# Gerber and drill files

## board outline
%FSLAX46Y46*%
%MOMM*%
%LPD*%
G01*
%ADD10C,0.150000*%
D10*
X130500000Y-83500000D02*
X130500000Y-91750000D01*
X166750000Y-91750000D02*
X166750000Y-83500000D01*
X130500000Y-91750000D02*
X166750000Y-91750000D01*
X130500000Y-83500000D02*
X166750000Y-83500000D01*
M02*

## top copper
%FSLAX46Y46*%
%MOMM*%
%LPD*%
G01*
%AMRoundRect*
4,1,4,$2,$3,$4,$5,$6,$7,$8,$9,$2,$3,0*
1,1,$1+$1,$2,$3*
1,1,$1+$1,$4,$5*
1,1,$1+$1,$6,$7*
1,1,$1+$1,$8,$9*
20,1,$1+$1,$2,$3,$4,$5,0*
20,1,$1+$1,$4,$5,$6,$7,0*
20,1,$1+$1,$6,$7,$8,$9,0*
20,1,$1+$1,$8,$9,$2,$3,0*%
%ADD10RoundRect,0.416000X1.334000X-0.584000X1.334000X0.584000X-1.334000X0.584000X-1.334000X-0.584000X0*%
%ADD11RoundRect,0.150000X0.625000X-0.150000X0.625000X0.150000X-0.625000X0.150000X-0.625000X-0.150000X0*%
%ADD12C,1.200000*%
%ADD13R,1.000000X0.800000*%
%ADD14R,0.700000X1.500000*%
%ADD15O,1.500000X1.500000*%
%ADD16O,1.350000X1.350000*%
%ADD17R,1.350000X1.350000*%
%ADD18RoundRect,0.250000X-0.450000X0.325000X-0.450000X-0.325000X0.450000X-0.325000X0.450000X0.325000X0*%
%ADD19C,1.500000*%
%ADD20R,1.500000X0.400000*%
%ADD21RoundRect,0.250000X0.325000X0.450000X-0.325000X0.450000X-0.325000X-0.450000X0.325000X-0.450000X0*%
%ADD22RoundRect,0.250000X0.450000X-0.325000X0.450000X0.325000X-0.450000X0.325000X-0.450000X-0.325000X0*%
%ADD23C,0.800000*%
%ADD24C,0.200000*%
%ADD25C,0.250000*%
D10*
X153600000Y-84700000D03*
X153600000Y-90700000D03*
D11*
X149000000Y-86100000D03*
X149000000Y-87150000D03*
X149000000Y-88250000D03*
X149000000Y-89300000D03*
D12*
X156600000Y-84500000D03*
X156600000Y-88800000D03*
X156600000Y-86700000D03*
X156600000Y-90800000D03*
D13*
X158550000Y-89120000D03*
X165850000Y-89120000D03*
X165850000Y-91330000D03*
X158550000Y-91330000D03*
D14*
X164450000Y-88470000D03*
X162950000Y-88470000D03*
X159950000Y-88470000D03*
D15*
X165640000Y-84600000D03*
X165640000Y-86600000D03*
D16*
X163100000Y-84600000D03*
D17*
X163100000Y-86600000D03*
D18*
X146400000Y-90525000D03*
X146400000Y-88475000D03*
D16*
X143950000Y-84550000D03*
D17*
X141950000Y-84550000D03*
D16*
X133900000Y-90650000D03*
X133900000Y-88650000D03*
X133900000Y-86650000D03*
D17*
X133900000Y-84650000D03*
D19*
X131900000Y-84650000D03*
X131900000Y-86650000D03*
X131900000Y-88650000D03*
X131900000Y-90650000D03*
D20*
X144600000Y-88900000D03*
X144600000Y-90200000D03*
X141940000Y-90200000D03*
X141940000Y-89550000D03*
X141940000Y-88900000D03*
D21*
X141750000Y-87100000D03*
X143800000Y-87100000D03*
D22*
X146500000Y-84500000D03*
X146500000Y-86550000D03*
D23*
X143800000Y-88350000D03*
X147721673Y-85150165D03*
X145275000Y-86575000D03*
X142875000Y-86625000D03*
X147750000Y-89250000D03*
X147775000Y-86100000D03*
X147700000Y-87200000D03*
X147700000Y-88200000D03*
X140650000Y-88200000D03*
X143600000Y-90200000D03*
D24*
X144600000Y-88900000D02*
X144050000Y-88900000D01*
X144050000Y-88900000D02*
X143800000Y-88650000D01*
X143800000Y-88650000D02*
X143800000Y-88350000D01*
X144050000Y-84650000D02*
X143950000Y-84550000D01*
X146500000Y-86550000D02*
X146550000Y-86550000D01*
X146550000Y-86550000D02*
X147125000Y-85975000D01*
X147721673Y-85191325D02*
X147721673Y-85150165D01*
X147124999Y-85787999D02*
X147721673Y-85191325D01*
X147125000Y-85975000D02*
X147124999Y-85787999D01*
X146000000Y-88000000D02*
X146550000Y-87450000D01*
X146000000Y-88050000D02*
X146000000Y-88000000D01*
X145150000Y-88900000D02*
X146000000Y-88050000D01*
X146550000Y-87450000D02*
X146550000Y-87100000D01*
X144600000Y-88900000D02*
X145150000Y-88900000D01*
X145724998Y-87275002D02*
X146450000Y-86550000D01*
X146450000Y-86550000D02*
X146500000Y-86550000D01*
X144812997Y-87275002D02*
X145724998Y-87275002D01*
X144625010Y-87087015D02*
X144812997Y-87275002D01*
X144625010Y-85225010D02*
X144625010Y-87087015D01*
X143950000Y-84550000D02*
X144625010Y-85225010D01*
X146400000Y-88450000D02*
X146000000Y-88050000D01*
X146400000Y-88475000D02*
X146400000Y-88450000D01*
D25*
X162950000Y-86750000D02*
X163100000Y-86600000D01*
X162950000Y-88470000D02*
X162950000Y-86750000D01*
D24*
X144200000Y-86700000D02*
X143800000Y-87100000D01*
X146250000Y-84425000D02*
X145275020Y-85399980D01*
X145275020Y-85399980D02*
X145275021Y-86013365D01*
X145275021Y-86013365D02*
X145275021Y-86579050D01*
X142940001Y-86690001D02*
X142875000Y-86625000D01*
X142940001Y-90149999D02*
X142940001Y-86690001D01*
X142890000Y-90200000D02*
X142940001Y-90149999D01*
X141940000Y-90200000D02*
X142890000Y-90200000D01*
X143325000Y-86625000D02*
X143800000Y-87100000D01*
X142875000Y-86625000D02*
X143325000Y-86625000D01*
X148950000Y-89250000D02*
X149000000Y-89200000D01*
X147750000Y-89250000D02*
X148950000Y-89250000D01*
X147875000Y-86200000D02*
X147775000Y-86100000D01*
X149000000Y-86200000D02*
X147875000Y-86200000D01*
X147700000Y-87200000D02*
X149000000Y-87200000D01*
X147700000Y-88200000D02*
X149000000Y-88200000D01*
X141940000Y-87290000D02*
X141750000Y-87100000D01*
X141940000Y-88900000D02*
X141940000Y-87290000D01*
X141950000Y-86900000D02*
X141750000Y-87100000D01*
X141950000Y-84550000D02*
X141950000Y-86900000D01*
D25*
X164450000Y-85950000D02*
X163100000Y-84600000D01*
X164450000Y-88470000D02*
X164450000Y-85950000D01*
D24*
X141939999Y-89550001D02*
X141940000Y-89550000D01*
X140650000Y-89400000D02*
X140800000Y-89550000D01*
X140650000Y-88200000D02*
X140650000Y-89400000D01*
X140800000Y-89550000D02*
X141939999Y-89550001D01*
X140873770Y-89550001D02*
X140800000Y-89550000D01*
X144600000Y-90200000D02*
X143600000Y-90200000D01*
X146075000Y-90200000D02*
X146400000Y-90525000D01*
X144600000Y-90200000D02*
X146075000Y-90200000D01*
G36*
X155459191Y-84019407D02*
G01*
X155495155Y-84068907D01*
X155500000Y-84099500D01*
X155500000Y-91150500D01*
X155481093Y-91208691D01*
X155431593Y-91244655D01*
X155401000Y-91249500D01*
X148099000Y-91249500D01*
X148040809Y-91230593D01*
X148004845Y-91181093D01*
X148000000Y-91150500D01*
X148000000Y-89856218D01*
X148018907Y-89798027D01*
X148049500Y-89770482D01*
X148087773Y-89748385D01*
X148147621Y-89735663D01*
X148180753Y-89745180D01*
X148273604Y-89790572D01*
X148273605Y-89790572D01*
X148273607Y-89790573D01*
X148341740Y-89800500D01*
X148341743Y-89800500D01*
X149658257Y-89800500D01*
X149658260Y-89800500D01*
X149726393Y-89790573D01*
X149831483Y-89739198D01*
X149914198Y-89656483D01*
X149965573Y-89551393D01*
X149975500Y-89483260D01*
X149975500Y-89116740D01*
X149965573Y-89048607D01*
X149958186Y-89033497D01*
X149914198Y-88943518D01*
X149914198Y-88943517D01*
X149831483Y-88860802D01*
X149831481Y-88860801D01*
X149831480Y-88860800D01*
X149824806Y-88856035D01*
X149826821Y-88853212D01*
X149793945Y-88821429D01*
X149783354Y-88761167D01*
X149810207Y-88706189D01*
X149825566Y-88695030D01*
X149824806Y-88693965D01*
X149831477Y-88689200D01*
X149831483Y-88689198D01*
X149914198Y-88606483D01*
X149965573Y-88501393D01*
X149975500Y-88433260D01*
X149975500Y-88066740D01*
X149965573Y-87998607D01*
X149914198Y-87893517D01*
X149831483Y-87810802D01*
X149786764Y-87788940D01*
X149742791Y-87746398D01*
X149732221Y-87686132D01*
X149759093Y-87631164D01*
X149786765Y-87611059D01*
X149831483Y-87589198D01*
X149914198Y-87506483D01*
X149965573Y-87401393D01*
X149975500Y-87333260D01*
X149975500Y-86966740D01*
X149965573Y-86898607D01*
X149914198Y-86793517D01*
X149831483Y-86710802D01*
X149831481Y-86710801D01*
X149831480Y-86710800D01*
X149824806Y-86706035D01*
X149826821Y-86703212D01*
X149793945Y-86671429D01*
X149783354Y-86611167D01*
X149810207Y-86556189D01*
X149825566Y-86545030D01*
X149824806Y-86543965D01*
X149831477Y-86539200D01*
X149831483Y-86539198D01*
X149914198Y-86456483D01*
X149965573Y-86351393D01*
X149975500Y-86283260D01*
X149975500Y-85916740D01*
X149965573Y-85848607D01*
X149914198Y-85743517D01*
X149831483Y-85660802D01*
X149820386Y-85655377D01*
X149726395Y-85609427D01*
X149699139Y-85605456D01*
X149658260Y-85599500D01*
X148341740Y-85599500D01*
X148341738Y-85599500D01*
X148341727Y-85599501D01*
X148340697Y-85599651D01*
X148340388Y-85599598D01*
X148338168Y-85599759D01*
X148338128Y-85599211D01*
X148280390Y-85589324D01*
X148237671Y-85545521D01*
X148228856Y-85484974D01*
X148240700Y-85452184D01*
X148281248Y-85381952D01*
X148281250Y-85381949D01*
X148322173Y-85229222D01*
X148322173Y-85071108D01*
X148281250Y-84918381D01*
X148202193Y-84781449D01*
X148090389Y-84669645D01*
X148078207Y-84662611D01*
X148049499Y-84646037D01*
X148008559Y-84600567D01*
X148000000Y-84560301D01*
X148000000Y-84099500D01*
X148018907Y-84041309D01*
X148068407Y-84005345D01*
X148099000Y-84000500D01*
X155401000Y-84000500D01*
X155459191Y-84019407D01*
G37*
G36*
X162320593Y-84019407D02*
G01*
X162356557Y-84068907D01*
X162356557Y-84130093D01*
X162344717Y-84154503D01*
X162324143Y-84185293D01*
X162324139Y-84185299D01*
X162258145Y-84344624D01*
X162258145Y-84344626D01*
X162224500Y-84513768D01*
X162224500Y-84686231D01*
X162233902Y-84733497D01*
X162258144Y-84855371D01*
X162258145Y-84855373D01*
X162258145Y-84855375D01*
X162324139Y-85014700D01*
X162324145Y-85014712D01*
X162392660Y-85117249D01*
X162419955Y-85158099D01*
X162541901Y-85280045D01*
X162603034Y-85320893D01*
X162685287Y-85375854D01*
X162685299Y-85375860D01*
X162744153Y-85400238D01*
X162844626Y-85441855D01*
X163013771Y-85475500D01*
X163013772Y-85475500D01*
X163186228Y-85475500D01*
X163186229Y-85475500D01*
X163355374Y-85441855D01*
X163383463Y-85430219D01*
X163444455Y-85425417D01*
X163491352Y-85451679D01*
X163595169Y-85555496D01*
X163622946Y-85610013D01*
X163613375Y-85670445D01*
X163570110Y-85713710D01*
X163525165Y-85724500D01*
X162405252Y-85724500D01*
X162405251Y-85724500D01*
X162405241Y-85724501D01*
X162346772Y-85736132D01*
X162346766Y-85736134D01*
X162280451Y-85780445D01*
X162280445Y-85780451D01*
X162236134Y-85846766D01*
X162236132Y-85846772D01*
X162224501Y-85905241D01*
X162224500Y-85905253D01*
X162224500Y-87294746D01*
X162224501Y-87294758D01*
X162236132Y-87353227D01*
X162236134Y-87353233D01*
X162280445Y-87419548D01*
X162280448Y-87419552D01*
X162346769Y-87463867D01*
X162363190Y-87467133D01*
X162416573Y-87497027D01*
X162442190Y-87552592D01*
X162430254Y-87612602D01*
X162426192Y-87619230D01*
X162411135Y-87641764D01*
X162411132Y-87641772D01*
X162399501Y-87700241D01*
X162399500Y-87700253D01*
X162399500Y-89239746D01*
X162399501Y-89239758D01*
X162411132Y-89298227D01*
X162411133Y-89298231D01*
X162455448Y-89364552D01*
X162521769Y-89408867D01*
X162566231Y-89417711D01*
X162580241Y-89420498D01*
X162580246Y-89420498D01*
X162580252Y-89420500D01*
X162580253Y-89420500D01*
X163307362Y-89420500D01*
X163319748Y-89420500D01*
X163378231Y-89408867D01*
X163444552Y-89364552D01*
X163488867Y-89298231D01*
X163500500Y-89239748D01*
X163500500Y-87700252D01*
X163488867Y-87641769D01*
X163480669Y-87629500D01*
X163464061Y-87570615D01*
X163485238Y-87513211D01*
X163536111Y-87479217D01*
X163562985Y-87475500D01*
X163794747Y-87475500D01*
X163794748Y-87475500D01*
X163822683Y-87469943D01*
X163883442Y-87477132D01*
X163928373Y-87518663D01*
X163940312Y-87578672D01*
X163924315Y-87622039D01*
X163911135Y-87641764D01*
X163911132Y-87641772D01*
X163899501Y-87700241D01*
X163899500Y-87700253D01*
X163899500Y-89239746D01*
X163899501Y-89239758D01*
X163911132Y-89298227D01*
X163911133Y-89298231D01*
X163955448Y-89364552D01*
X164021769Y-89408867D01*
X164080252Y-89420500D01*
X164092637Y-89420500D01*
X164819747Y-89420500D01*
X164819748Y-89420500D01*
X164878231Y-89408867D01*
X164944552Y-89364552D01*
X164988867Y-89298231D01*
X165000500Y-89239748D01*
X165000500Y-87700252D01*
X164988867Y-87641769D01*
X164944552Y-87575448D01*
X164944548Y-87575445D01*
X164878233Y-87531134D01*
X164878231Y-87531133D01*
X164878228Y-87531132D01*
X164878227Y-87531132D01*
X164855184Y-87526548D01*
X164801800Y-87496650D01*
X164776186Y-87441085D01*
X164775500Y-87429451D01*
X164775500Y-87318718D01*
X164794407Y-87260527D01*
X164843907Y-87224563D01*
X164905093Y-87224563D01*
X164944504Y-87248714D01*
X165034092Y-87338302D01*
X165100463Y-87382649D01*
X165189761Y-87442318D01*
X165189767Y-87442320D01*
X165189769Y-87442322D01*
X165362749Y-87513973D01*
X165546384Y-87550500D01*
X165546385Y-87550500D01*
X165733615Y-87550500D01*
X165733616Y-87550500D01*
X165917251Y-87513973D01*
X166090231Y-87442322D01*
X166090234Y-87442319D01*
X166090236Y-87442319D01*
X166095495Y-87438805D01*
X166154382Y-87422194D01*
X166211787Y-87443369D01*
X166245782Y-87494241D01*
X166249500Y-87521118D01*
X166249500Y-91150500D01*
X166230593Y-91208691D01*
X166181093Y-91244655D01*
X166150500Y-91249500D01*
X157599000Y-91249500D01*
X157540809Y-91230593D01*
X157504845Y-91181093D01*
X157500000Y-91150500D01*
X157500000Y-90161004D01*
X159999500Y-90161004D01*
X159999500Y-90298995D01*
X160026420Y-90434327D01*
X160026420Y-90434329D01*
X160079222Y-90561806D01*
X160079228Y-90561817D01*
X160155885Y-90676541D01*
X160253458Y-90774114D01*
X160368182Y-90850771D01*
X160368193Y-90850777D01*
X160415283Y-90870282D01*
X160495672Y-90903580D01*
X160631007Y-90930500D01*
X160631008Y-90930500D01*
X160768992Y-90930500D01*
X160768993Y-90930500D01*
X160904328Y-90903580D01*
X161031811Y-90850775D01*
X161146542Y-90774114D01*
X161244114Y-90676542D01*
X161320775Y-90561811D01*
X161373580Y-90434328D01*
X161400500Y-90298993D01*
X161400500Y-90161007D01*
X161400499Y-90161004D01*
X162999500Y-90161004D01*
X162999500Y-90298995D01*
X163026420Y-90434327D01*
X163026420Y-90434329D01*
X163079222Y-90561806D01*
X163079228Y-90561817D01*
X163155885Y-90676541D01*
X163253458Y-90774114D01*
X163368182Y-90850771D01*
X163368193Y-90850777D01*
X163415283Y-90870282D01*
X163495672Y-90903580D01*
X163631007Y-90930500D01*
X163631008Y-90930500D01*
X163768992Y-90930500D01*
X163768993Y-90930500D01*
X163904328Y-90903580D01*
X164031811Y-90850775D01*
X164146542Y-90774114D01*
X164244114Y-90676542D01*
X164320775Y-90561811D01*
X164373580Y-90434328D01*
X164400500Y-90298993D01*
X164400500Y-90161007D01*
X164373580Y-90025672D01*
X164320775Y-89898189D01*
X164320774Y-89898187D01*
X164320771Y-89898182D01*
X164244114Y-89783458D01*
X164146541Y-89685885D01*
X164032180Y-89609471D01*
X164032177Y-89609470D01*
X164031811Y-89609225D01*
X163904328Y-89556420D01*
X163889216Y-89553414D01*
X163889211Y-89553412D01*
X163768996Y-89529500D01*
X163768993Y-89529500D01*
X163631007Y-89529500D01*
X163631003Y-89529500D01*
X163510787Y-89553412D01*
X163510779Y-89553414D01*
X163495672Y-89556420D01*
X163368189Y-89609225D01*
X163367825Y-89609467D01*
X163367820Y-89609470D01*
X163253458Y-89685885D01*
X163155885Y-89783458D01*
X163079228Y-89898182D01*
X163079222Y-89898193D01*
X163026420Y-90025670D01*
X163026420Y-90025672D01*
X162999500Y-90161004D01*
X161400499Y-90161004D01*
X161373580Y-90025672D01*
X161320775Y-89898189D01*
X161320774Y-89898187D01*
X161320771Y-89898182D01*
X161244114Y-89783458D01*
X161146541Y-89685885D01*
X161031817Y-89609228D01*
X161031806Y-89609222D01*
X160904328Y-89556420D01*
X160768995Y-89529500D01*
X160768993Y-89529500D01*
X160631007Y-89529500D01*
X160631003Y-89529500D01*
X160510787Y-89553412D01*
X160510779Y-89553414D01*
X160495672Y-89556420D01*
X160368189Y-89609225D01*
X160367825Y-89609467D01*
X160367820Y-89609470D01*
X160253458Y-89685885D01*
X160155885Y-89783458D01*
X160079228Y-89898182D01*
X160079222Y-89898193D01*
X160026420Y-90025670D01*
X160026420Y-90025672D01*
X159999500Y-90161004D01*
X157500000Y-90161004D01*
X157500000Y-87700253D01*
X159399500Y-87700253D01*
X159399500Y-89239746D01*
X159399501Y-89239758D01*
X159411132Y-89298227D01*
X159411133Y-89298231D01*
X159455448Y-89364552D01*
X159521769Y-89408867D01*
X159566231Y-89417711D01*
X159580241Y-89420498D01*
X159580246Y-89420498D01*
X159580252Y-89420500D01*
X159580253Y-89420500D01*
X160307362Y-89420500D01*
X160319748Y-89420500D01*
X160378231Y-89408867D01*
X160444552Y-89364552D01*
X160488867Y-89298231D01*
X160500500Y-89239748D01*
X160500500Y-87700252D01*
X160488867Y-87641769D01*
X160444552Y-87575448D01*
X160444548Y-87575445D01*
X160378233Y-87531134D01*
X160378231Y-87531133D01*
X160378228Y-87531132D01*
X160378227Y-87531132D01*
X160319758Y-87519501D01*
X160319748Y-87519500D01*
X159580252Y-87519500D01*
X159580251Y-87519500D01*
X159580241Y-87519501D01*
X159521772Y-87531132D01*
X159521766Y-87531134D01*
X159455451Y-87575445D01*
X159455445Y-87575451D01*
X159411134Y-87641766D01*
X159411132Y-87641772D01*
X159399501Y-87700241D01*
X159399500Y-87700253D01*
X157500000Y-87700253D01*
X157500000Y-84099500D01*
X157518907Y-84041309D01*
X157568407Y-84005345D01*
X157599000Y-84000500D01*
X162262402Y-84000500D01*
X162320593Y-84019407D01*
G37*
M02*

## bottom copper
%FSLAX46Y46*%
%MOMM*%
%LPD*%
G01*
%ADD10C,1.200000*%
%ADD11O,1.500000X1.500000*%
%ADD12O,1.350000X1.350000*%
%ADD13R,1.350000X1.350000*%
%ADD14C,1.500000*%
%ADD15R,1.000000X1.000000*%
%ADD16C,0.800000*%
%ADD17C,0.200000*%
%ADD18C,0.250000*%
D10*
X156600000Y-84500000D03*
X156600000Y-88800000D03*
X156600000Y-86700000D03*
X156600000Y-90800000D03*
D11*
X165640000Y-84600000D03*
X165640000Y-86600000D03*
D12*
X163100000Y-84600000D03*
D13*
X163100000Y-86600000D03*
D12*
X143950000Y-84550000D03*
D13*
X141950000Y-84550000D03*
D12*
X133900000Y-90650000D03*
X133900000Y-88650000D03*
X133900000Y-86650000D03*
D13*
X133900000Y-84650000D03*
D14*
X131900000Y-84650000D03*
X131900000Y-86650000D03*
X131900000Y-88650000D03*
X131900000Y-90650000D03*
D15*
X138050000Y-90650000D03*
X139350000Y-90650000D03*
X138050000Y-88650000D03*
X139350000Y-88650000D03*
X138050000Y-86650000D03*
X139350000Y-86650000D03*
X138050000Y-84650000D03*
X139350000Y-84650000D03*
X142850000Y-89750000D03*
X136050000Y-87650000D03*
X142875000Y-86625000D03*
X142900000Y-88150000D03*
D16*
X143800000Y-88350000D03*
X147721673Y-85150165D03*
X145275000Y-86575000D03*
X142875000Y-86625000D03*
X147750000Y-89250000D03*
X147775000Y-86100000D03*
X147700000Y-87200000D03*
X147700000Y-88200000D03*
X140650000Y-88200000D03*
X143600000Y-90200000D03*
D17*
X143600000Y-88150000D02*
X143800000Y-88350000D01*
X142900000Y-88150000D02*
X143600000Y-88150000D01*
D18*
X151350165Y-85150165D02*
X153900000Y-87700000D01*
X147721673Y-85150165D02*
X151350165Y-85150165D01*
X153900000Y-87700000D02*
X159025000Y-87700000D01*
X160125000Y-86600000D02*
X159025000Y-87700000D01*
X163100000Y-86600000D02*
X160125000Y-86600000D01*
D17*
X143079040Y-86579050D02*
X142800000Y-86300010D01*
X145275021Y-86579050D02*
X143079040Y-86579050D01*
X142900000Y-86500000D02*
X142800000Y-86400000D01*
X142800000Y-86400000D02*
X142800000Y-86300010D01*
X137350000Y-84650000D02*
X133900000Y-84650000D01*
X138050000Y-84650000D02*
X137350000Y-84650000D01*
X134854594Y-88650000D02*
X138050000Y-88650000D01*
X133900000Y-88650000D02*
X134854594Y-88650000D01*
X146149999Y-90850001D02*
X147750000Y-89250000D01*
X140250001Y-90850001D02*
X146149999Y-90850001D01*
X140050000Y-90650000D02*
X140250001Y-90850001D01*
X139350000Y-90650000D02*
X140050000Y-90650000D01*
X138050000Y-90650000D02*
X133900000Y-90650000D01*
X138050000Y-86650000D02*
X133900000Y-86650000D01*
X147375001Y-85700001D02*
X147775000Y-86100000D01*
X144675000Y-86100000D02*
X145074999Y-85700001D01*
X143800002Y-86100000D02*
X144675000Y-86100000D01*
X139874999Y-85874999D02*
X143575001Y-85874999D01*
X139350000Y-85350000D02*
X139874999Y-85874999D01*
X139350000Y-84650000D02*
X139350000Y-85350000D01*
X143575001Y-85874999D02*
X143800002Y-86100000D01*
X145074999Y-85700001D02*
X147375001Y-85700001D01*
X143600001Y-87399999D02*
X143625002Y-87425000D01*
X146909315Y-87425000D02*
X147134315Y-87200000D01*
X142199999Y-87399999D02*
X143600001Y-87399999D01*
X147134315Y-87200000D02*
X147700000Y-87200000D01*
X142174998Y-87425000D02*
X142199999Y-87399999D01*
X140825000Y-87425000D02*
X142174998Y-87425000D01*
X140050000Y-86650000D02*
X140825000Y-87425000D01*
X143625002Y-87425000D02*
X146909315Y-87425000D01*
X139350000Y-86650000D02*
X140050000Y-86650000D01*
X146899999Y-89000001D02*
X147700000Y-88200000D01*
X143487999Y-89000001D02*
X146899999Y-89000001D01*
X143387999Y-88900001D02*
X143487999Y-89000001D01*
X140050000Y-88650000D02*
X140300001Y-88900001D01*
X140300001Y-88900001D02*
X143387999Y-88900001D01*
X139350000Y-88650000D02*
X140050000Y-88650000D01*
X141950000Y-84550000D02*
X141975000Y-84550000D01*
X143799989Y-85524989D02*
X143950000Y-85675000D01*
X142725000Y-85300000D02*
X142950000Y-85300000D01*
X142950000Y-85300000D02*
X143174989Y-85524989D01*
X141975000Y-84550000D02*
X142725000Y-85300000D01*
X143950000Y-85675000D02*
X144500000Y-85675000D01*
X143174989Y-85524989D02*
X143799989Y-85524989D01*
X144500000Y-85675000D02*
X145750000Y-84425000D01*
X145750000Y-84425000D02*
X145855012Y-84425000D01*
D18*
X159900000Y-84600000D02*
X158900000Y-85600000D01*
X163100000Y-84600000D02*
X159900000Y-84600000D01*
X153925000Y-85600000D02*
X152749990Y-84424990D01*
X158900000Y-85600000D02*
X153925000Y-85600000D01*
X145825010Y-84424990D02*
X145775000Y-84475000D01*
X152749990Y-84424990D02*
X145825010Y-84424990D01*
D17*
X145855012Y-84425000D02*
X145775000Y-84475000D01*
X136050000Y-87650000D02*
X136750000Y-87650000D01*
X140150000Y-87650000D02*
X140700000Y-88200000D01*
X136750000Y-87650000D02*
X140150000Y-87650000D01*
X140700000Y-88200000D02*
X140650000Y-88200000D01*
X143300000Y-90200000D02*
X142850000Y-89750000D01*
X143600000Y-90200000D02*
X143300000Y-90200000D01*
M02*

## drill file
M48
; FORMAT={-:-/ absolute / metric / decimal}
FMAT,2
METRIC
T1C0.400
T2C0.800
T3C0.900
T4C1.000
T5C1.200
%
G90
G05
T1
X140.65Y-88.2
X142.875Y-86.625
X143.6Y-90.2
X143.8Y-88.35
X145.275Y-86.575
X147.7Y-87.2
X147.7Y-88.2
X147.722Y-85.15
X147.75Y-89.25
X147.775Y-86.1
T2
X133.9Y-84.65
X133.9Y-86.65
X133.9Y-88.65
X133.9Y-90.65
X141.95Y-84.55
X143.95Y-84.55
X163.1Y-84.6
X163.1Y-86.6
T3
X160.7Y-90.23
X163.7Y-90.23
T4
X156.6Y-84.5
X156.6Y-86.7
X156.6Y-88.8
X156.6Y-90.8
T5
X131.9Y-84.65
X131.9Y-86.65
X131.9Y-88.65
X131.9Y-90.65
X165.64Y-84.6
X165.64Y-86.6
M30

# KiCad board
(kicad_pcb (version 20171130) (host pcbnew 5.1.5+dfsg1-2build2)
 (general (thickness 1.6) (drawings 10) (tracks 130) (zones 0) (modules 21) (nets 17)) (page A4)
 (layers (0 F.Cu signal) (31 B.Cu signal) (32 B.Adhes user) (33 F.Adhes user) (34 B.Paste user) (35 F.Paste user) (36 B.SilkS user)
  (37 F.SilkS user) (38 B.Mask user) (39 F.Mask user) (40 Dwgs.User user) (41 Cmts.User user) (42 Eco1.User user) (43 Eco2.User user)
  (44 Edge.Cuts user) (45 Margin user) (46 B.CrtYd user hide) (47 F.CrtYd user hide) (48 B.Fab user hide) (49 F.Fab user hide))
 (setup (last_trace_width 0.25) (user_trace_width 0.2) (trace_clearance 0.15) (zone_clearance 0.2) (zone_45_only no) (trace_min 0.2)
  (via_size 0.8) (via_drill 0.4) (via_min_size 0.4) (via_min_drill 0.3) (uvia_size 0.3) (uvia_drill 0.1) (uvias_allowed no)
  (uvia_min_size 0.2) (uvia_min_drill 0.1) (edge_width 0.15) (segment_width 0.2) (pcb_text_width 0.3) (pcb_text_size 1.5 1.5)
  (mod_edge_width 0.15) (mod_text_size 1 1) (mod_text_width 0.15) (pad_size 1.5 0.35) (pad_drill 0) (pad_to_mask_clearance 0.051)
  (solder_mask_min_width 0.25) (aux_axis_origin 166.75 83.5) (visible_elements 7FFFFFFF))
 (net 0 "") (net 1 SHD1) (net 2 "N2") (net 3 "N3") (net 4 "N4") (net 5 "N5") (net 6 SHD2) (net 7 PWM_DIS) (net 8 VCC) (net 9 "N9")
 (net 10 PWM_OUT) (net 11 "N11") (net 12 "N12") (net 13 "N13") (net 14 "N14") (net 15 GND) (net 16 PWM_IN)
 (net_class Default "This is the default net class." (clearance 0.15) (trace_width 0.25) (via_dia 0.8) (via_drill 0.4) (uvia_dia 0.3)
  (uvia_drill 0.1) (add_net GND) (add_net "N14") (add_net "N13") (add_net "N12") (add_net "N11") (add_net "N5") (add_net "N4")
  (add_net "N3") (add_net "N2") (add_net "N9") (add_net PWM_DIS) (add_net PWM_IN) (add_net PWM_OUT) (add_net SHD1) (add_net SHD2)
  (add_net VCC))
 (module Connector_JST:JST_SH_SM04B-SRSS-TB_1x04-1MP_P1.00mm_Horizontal (layer F.Cu) (at 151 87.7 90)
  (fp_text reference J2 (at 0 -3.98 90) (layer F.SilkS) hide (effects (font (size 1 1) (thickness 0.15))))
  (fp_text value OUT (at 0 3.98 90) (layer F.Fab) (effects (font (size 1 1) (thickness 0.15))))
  (pad MP smd roundrect (at 3 2.6 90) (size 2 3.5) (layers F.Cu F.Paste F.Mask) (roundrect_rratio 0.208) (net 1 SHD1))
  (pad MP smd roundrect (at -3 2.6 90) (size 2 3.5) (layers F.Cu F.Paste F.Mask) (roundrect_rratio 0.208) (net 1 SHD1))
  (pad 4 smd roundrect (at 1.6 -2 90) (size 0.6 1.55) (layers F.Cu F.Paste F.Mask) (roundrect_rratio 0.25) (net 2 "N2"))
  (pad 3 smd roundrect (at 0.55 -2 90) (size 0.6 1.55) (layers F.Cu F.Paste F.Mask) (roundrect_rratio 0.25) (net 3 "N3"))
  (pad 2 smd roundrect (at -0.55 -2 90) (size 0.6 1.55) (layers F.Cu F.Paste F.Mask) (roundrect_rratio 0.25) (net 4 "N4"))
  (pad 1 smd roundrect (at -1.6 -2 90) (size 0.6 1.55) (layers F.Cu F.Paste F.Mask) (roundrect_rratio 0.25) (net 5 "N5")))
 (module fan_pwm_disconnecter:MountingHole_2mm (layer F.Cu) (at 156.6 84.5)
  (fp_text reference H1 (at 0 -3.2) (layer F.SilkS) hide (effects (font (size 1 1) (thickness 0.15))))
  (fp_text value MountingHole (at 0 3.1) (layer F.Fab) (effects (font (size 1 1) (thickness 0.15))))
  (pad "" np_thru_hole circle (at 0 0) (size 1.2 1.2) (drill 1) (layers *.Cu *.Mask)))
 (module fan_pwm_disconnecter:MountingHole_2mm (layer F.Cu) (at 156.6 88.8)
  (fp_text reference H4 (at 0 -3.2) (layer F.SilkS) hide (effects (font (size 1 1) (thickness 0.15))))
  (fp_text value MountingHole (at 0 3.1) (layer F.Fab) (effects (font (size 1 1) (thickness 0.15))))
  (pad "" np_thru_hole circle (at 0 0) (size 1.2 1.2) (drill 1) (layers *.Cu *.Mask)))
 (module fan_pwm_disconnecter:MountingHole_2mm (layer F.Cu) (at 156.6 86.7)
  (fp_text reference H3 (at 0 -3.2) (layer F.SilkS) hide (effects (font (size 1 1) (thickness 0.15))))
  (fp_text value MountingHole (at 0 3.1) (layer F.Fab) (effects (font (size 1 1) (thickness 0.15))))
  (pad "" np_thru_hole circle (at 0 0) (size 1.2 1.2) (drill 1) (layers *.Cu *.Mask)))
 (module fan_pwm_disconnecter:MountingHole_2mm (layer F.Cu) (at 156.6 90.8)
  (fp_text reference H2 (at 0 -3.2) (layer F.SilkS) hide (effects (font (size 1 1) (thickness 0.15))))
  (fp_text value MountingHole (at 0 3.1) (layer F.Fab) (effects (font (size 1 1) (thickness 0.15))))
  (pad "" np_thru_hole circle (at 0 0) (size 1.2 1.2) (drill 1) (layers *.Cu *.Mask)))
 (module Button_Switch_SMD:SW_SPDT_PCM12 (layer F.Cu) (at 162.2 89.9)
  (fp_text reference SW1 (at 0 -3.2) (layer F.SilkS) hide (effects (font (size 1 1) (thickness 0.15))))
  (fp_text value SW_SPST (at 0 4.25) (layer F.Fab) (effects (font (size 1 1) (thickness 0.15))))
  (pad 4 smd rect (at -3.65 -0.78) (size 1 0.8) (layers F.Cu F.Paste F.Mask) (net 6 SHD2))
  (pad 4 smd rect (at 3.65 -0.78) (size 1 0.8) (layers F.Cu F.Paste F.Mask) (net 6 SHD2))
  (pad 4 smd rect (at 3.65 1.43) (size 1 0.8) (layers F.Cu F.Paste F.Mask) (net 6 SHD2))
  (pad 4 smd rect (at -3.65 1.43) (size 1 0.8) (layers F.Cu F.Paste F.Mask) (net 6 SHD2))
  (pad 3 smd rect (at 2.25 -1.43) (size 0.7 1.5) (layers F.Cu F.Paste F.Mask) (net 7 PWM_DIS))
  (pad 2 smd rect (at 0.75 -1.43) (size 0.7 1.5) (layers F.Cu F.Paste F.Mask) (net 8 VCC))
  (pad 1 smd rect (at -2.25 -1.43) (size 0.7 1.5) (layers F.Cu F.Paste F.Mask) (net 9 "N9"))
  (pad "" np_thru_hole circle (at 1.5 0.33) (size 0.9 0.9) (drill 0.9) (layers *.Cu *.Mask))
  (pad "" np_thru_hole circle (at -1.5 0.33) (size 0.9 0.9) (drill 0.9) (layers *.Cu *.Mask)))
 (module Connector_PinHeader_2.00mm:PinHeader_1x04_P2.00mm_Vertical (layer F.Cu) (at 163.1 86.6 180)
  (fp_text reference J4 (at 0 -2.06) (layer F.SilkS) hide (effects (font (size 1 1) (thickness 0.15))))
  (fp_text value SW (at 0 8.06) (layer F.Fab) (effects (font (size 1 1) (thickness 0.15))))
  (pad "" np_thru_hole oval (at -2.54 2 180) (size 1.5 1.5) (drill 1.2) (layers *.Cu *.Mask))
  (pad "" np_thru_hole oval (at -2.54 0 180) (size 1.5 1.5) (drill 1.2) (layers *.Cu *.Mask))
  (pad 2 thru_hole oval (at 0 2 180) (size 1.35 1.35) (drill 0.8) (layers *.Cu *.Mask) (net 7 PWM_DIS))
  (pad 1 thru_hole rect (at 0 0 180) (size 1.35 1.35) (drill 0.8) (layers *.Cu *.Mask) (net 8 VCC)))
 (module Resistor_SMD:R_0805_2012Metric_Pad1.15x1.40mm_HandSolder (layer F.Cu) (at 146.4 89.5 270)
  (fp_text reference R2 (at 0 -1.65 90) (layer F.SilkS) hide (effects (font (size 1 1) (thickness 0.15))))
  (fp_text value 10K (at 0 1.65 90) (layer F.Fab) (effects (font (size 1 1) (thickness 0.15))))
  (pad 2 smd roundrect (at 1.025 0 270) (size 1.15 1.4) (layers F.Cu F.Paste F.Mask) (roundrect_rratio 0.217391) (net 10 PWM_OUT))
  (pad 1 smd roundrect (at -1.025 0 270) (size 1.15 1.4) (layers F.Cu F.Paste F.Mask) (roundrect_rratio 0.217391) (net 8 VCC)))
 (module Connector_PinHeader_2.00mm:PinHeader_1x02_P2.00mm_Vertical (layer F.Cu) (at 141.95 84.55 90)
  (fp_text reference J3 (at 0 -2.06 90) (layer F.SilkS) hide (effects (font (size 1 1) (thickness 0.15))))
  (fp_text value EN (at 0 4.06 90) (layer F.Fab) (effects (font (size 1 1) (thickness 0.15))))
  (pad 2 thru_hole oval (at 0 2 90) (size 1.35 1.35) (drill 0.8) (layers *.Cu *.Mask) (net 8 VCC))
  (pad 1 thru_hole rect (at 0 0 90) (size 1.35 1.35) (drill 0.8) (layers *.Cu *.Mask) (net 7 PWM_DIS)))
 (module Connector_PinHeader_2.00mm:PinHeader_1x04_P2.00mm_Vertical (layer F.Cu) (at 133.9 84.65)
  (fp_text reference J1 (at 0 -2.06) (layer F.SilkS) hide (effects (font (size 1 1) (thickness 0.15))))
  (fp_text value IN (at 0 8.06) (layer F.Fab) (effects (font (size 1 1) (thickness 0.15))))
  (pad 4 thru_hole oval (at 0 6) (size 1.35 1.35) (drill 0.8) (layers *.Cu *.Mask) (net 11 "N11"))
  (pad 3 thru_hole oval (at 0 4) (size 1.35 1.35) (drill 0.8) (layers *.Cu *.Mask) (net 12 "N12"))
  (pad 2 thru_hole oval (at 0 2) (size 1.35 1.35) (drill 0.8) (layers *.Cu *.Mask) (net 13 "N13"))
  (pad 1 thru_hole rect (at 0 0) (size 1.35 1.35) (drill 0.8) (layers *.Cu *.Mask) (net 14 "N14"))
  (pad "" np_thru_hole circle (at -2 0) (size 1.5 1.5) (drill 1.2) (layers *.Cu *.Mask))
  (pad "" np_thru_hole circle (at -2 2) (size 1.5 1.5) (drill 1.2) (layers *.Cu *.Mask))
  (pad "" np_thru_hole circle (at -2 4) (size 1.5 1.5) (drill 1.2) (layers *.Cu *.Mask))
  (pad "" np_thru_hole circle (at -2 6) (size 1.5 1.5) (drill 1.2) (layers *.Cu *.Mask)))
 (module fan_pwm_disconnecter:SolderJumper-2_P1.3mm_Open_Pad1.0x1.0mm (layer B.Cu) (at 138.7 90.65)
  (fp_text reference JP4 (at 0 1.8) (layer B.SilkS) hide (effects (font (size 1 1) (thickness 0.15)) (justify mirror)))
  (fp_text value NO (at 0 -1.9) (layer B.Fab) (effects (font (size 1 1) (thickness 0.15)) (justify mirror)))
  (pad 1 smd rect (at -0.65 0) (size 1 1) (layers B.Cu B.Mask) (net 11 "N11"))
  (pad 2 smd rect (at 0.65 0) (size 1 1) (layers B.Cu B.Mask) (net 5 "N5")))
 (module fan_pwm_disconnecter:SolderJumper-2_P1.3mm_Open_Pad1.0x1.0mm (layer B.Cu) (at 138.7 88.65)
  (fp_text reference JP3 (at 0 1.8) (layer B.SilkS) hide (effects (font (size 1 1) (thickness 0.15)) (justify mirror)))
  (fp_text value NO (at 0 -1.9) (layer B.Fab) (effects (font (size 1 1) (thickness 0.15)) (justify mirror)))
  (pad 1 smd rect (at -0.65 0) (size 1 1) (layers B.Cu B.Mask) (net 12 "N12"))
  (pad 2 smd rect (at 0.65 0) (size 1 1) (layers B.Cu B.Mask) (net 4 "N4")))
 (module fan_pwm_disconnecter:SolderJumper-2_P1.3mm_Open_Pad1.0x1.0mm (layer B.Cu) (at 138.7 86.65)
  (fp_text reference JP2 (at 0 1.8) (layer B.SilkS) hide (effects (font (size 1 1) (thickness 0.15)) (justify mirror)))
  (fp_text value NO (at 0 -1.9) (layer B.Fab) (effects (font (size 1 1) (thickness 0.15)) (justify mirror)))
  (pad 1 smd rect (at -0.65 0) (size 1 1) (layers B.Cu B.Mask) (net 13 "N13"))
  (pad 2 smd rect (at 0.65 0) (size 1 1) (layers B.Cu B.Mask) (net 3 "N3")))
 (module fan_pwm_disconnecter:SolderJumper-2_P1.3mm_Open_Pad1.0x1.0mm (layer B.Cu) (at 138.7 84.65)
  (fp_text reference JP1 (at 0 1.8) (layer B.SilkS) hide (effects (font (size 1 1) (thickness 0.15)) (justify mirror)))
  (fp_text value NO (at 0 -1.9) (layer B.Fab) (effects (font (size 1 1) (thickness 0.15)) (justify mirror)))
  (pad 1 smd rect (at -0.65 0) (size 1 1) (layers B.Cu B.Mask) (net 14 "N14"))
  (pad 2 smd rect (at 0.65 0) (size 1 1) (layers B.Cu B.Mask) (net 2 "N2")))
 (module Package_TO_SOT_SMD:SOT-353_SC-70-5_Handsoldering (layer F.Cu) (at 143.27 89.55)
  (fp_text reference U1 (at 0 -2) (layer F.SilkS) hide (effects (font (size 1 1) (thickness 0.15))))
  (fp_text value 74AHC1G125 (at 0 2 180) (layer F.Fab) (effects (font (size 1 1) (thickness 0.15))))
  (pad 5 smd rect (at 1.33 -0.65) (size 1.5 0.4) (layers F.Cu F.Paste F.Mask) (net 8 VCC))
  (pad 4 smd rect (at 1.33 0.65) (size 1.5 0.4) (layers F.Cu F.Paste F.Mask) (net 10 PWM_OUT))
  (pad 3 smd rect (at -1.33 0.65) (size 1.5 0.4) (layers F.Cu F.Paste F.Mask) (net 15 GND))
  (pad 2 smd rect (at -1.33 0) (size 1.5 0.4) (layers F.Cu F.Paste F.Mask) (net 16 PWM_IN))
  (pad 1 smd rect (at -1.33 -0.65) (size 1.5 0.4) (layers F.Cu F.Paste F.Mask) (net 7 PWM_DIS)))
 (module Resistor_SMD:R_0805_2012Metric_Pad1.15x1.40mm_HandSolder (layer F.Cu) (at 142.775 87.1 180)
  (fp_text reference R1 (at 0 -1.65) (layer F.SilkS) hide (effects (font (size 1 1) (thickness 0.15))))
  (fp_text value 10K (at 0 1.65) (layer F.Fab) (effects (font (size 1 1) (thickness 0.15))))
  (pad 2 smd roundrect (at 1.025 0 180) (size 1.15 1.4) (layers F.Cu F.Paste F.Mask) (roundrect_rratio 0.217391) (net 7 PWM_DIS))
  (pad 1 smd roundrect (at -1.025 0 180) (size 1.15 1.4) (layers F.Cu F.Paste F.Mask) (roundrect_rratio 0.217391) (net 15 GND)))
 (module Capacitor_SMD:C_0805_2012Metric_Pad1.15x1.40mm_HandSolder (layer F.Cu) (at 146.5 85.525 90)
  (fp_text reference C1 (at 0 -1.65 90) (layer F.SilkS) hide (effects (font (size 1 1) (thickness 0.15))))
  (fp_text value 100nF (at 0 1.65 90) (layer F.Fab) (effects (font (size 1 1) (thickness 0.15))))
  (pad 2 smd roundrect (at 1.025 0 90) (size 1.15 1.4) (layers F.Cu F.Paste F.Mask) (roundrect_rratio 0.217391) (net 15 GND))
  (pad 1 smd roundrect (at -1.025 0 90) (size 1.15 1.4) (layers F.Cu F.Paste F.Mask) (roundrect_rratio 0.217391) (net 8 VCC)))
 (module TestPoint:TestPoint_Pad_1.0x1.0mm (layer B.Cu) (at 142.85 89.75)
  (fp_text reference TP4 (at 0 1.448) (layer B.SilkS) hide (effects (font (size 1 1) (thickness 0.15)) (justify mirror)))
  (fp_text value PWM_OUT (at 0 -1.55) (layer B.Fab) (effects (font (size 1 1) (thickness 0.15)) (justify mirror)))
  (pad 1 smd rect (at 0 0) (size 1 1) (layers B.Cu B.Mask) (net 10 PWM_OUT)))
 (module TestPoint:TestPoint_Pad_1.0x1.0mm (layer B.Cu) (at 136.05 87.65)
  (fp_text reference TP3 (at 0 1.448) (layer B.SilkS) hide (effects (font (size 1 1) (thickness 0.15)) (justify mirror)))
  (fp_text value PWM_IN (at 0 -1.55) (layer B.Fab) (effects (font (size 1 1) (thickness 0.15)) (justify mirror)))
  (pad 1 smd rect (at 0 0) (size 1 1) (layers B.Cu B.Mask) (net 16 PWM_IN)))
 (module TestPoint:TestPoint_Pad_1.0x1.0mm (layer B.Cu) (at 142.875 86.625)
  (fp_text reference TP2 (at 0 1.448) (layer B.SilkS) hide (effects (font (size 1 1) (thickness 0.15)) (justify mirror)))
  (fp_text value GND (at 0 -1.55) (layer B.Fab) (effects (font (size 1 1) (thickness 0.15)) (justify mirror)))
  (pad 1 smd rect (at 0 0) (size 1 1) (layers B.Cu B.Mask) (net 15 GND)))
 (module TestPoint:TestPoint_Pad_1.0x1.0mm (layer B.Cu) (at 142.9 88.15)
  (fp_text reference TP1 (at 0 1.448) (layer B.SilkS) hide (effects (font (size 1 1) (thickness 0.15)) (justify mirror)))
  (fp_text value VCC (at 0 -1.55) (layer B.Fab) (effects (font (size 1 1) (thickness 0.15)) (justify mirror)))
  (pad 1 smd rect (at 0 0) (size 1 1) (layers B.Cu B.Mask) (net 8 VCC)))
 (gr_line (start 130.5 83.5) (end 130.5 91.75) (layer Edge.Cuts) (width 0.15))
 (gr_line (start 166.75 91.75) (end 166.75 83.5) (layer Edge.Cuts) (width 0.15))
 (gr_line (start 130.5 91.75) (end 166.75 91.75) (layer Edge.Cuts) (width 0.15))
 (gr_line (start 130.5 83.5) (end 166.75 83.5) (layer Edge.Cuts) (width 0.15))
 (segment (start 144.6 88.9) (end 144.05 88.9) (width 0.2) (layer F.Cu) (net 8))
 (segment (start 144.05 88.9) (end 143.8 88.65) (width 0.2) (layer F.Cu) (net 8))
 (segment (start 143.6 88.15) (end 143.8 88.35) (width 0.2) (layer B.Cu) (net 8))
 (segment (start 142.9 88.15) (end 143.6 88.15) (width 0.2) (layer B.Cu) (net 8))
 (via (at 143.8 88.35) (size 0.8) (drill 0.4) (layers F.Cu B.Cu) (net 8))
 (segment (start 143.8 88.65) (end 143.8 88.35) (width 0.2) (layer F.Cu) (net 8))
 (segment (start 144.05 84.65) (end 143.95 84.55) (width 0.2) (layer F.Cu) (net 8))
 (segment (start 146.5 86.55) (end 146.55 86.55) (width 0.2) (layer F.Cu) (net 8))
 (segment (start 146.55 86.55) (end 147.125 85.975) (width 0.2) (layer F.Cu) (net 8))
 (via (at 147.721673 85.150165) (size 0.8) (drill 0.4) (layers F.Cu B.Cu) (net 8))
 (segment (start 147.721673 85.191325) (end 147.721673 85.150165) (width 0.2) (layer F.Cu) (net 8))
 (segment (start 147.124999 85.787999) (end 147.721673 85.191325) (width 0.2) (layer F.Cu) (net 8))
 (segment (start 147.125 85.975) (end 147.124999 85.787999) (width 0.2) (layer F.Cu) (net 8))
 (segment (start 146 88) (end 146.55 87.45) (width 0.2) (layer F.Cu) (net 8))
 (segment (start 146 88.05) (end 146 88) (width 0.2) (layer F.Cu) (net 8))
 (segment (start 145.15 88.9) (end 146 88.05) (width 0.2) (layer F.Cu) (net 8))
 (segment (start 146.55 87.45) (end 146.55 87.1) (width 0.2) (layer F.Cu) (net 8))
 (segment (start 144.6 88.9) (end 145.15 88.9) (width 0.2) (layer F.Cu) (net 8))
 (segment (start 145.724998 87.275002) (end 146.45 86.55) (width 0.2) (layer F.Cu) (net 8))
 (segment (start 146.45 86.55) (end 146.5 86.55) (width 0.2) (layer F.Cu) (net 8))
 (segment (start 144.812997 87.275002) (end 145.724998 87.275002) (width 0.2) (layer F.Cu) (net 8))
 (segment (start 144.62501 87.087015) (end 144.812997 87.275002) (width 0.2) (layer F.Cu) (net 8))
 (segment (start 144.62501 85.22501) (end 144.62501 87.087015) (width 0.2) (layer F.Cu) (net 8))
 (segment (start 143.95 84.55) (end 144.62501 85.22501) (width 0.2) (layer F.Cu) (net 8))
 (segment (start 146.4 88.45) (end 146 88.05) (width 0.2) (layer F.Cu) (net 8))
 (segment (start 146.4 88.475) (end 146.4 88.45) (width 0.2) (layer F.Cu) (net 8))
 (segment (start 162.95 86.75) (end 163.1 86.6) (width 0.25) (layer F.Cu) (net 8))
 (segment (start 162.95 88.47) (end 162.95 86.75) (width 0.25) (layer F.Cu) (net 8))
 (segment (start 151.350165 85.150165) (end 153.9 87.7) (width 0.25) (layer B.Cu) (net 8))
 (segment (start 147.721673 85.150165) (end 151.350165 85.150165) (width 0.25) (layer B.Cu) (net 8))
 (segment (start 153.9 87.7) (end 159.025 87.7) (width 0.25) (layer B.Cu) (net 8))
 (segment (start 160.125 86.6) (end 159.025 87.7) (width 0.25) (layer B.Cu) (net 8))
 (segment (start 163.1 86.6) (end 160.125 86.6) (width 0.25) (layer B.Cu) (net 8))
 (segment (start 144.2 86.7) (end 143.8 87.1) (width 0.2) (layer F.Cu) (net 15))
 (segment (start 146.25 84.425) (end 145.27502 85.39998) (width 0.2) (layer F.Cu) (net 15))
 (segment (start 145.27502 85.39998) (end 145.275021 86.013365) (width 0.2) (layer F.Cu) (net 15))
 (via (at 145.275 86.575) (size 0.8) (drill 0.4) (layers F.Cu B.Cu) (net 15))
 (segment (start 145.275021 86.013365) (end 145.275021 86.57905) (width 0.2) (layer F.Cu) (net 15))
 (segment (start 143.07904 86.57905) (end 142.8 86.30001) (width 0.2) (layer B.Cu) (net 15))
 (segment (start 145.275021 86.57905) (end 143.07904 86.57905) (width 0.2) (layer B.Cu) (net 15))
 (segment (start 142.9 86.5) (end 142.8 86.4) (width 0.2) (layer B.Cu) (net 15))
 (segment (start 142.8 86.4) (end 142.8 86.30001) (width 0.2) (layer B.Cu) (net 15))
 (segment (start 142.940001 86.690001) (end 142.875 86.625) (width 0.2) (layer F.Cu) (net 15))
 (segment (start 142.940001 90.149999) (end 142.940001 86.690001) (width 0.2) (layer F.Cu) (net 15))
 (segment (start 142.89 90.2) (end 142.940001 90.149999) (width 0.2) (layer F.Cu) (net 15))
 (segment (start 141.94 90.2) (end 142.89 90.2) (width 0.2) (layer F.Cu) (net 15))
 (via (at 142.875 86.625) (size 0.8) (drill 0.4) (layers F.Cu B.Cu) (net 15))
 (segment (start 143.325 86.625) (end 143.8 87.1) (width 0.2) (layer F.Cu) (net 15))
 (segment (start 142.875 86.625) (end 143.325 86.625) (width 0.2) (layer F.Cu) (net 15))
 (segment (start 137.35 84.65) (end 133.9 84.65) (width 0.2) (layer B.Cu) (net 14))
 (segment (start 138.05 84.65) (end 137.35 84.65) (width 0.2) (layer B.Cu) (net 14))
 (segment (start 134.854594 88.65) (end 138.05 88.65) (width 0.2) (layer B.Cu) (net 12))
 (segment (start 133.9 88.65) (end 134.854594 88.65) (width 0.2) (layer B.Cu) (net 12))
 (segment (start 146.149999 90.850001) (end 147.75 89.25) (width 0.2) (layer B.Cu) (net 5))
 (via (at 147.75 89.25) (size 0.8) (drill 0.4) (layers F.Cu B.Cu) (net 5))
 (segment (start 140.250001 90.850001) (end 146.149999 90.850001) (width 0.2) (layer B.Cu) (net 5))
 (segment (start 140.05 90.65) (end 140.250001 90.850001) (width 0.2) (layer B.Cu) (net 5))
 (segment (start 139.35 90.65) (end 140.05 90.65) (width 0.2) (layer B.Cu) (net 5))
 (segment (start 148.95 89.25) (end 149 89.2) (width 0.2) (layer F.Cu) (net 5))
 (segment (start 147.75 89.25) (end 148.95 89.25) (width 0.2) (layer F.Cu) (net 5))
 (segment (start 138.05 90.65) (end 133.9 90.65) (width 0.2) (layer B.Cu) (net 11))
 (segment (start 138.05 86.65) (end 133.9 86.65) (width 0.2) (layer B.Cu) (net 13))
 (segment (start 147.375001 85.700001) (end 147.775 86.1) (width 0.2) (layer B.Cu) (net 2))
 (segment (start 144.675 86.1) (end 145.074999 85.700001) (width 0.2) (layer B.Cu) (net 2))
 (segment (start 143.800002 86.1) (end 144.675 86.1) (width 0.2) (layer B.Cu) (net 2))
 (segment (start 139.874999 85.874999) (end 143.575001 85.874999) (width 0.2) (layer B.Cu) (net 2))
 (segment (start 139.35 85.35) (end 139.874999 85.874999) (width 0.2) (layer B.Cu) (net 2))
 (segment (start 139.35 84.65) (end 139.35 85.35) (width 0.2) (layer B.Cu) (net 2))
 (segment (start 143.575001 85.874999) (end 143.800002 86.1) (width 0.2) (layer B.Cu) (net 2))
 (segment (start 147.875 86.2) (end 147.775 86.1) (width 0.2) (layer F.Cu) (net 2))
 (segment (start 149 86.2) (end 147.875 86.2) (width 0.2) (layer F.Cu) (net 2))
 (segment (start 145.074999 85.700001) (end 147.375001 85.700001) (width 0.2) (layer B.Cu) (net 2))
 (via (at 147.775 86.1) (size 0.8) (drill 0.4) (layers F.Cu B.Cu) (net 2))
 (via (at 147.7 87.2) (size 0.8) (drill 0.4) (layers F.Cu B.Cu) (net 3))
 (segment (start 147.7 87.2) (end 149 87.2) (width 0.2) (layer F.Cu) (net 3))
 (segment (start 143.600001 87.399999) (end 143.625002 87.425) (width 0.2) (layer B.Cu) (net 3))
 (segment (start 146.909315 87.425) (end 147.134315 87.2) (width 0.2) (layer B.Cu) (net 3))
 (segment (start 142.199999 87.399999) (end 143.600001 87.399999) (width 0.2) (layer B.Cu) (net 3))
 (segment (start 147.134315 87.2) (end 147.7 87.2) (width 0.2) (layer B.Cu) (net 3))
 (segment (start 142.174998 87.425) (end 142.199999 87.399999) (width 0.2) (layer B.Cu) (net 3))
 (segment (start 140.825 87.425) (end 142.174998 87.425) (width 0.2) (layer B.Cu) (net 3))
 (segment (start 140.05 86.65) (end 140.825 87.425) (width 0.2) (layer B.Cu) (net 3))
 (segment (start 143.625002 87.425) (end 146.909315 87.425) (width 0.2) (layer B.Cu) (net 3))
 (segment (start 139.35 86.65) (end 140.05 86.65) (width 0.2) (layer B.Cu) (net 3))
 (via (at 147.7 88.2) (size 0.8) (drill 0.4) (layers F.Cu B.Cu) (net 4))
 (segment (start 146.899999 89.000001) (end 147.7 88.2) (width 0.2) (layer B.Cu) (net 4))
 (segment (start 143.487999 89.000001) (end 146.899999 89.000001) (width 0.2) (layer B.Cu) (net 4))
 (segment (start 143.387999 88.900001) (end 143.487999 89.000001) (width 0.2) (layer B.Cu) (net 4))
 (segment (start 140.05 88.65) (end 140.300001 88.900001) (width 0.2) (layer B.Cu) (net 4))
 (segment (start 140.300001 88.900001) (end 143.387999 88.900001) (width 0.2) (layer B.Cu) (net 4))
 (segment (start 139.35 88.65) (end 140.05 88.65) (width 0.2) (layer B.Cu) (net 4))
 (segment (start 147.7 88.2) (end 149 88.2) (width 0.2) (layer F.Cu) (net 4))
 (segment (start 141.94 87.29) (end 141.75 87.1) (width 0.2) (layer F.Cu) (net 7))
 (segment (start 141.94 88.9) (end 141.94 87.29) (width 0.2) (layer F.Cu) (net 7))
 (segment (start 141.95 86.9) (end 141.75 87.1) (width 0.2) (layer F.Cu) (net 7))
 (segment (start 141.95 84.55) (end 141.95 86.9) (width 0.2) (layer F.Cu) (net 7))
 (segment (start 141.95 84.55) (end 141.975 84.55) (width 0.2) (layer B.Cu) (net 7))
 (segment (start 143.799989 85.524989) (end 143.95 85.675) (width 0.2) (layer B.Cu) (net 7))
 (segment (start 142.725 85.3) (end 142.95 85.3) (width 0.2) (layer B.Cu) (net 7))
 (segment (start 142.95 85.3) (end 143.174989 85.524989) (width 0.2) (layer B.Cu) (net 7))
 (segment (start 141.975 84.55) (end 142.725 85.3) (width 0.2) (layer B.Cu) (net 7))
 (segment (start 143.95 85.675) (end 144.5 85.675) (width 0.2) (layer B.Cu) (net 7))
 (segment (start 143.174989 85.524989) (end 143.799989 85.524989) (width 0.2) (layer B.Cu) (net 7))
 (segment (start 144.5 85.675) (end 145.75 84.425) (width 0.2) (layer B.Cu) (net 7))
 (segment (start 145.75 84.425) (end 145.855012 84.425) (width 0.2) (layer B.Cu) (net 7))
 (segment (start 164.45 85.95) (end 163.1 84.6) (width 0.25) (layer F.Cu) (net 7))
 (segment (start 164.45 88.47) (end 164.45 85.95) (width 0.25) (layer F.Cu) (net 7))
 (segment (start 159.9 84.6) (end 158.9 85.6) (width 0.25) (layer B.Cu) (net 7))
 (segment (start 163.1 84.6) (end 159.9 84.6) (width 0.25) (layer B.Cu) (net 7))
 (segment (start 153.925 85.6) (end 152.74999 84.42499) (width 0.25) (layer B.Cu) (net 7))
 (segment (start 158.9 85.6) (end 153.925 85.6) (width 0.25) (layer B.Cu) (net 7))
 (segment (start 145.82501 84.42499) (end 145.775 84.475) (width 0.25) (layer B.Cu) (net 7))
 (segment (start 152.74999 84.42499) (end 145.82501 84.42499) (width 0.25) (layer B.Cu) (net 7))
 (segment (start 145.855012 84.425) (end 145.775 84.475) (width 0.2) (layer B.Cu) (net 7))
 (segment (start 136.05 87.65) (end 136.75 87.65) (width 0.2) (layer B.Cu) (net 16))
 (segment (start 141.939999 89.550001) (end 141.94 89.55) (width 0.2) (layer F.Cu) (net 16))
 (segment (start 140.15 87.65) (end 140.7 88.2) (width 0.2) (layer B.Cu) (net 16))
 (segment (start 136.75 87.65) (end 140.15 87.65) (width 0.2) (layer B.Cu) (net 16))
 (via (at 140.65 88.2) (size 0.8) (drill 0.4) (layers F.Cu B.Cu) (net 16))
 (segment (start 140.7 88.2) (end 140.65 88.2) (width 0.2) (layer B.Cu) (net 16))
 (segment (start 140.65 89.4) (end 140.8 89.55) (width 0.2) (layer F.Cu) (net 16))
 (segment (start 140.65 88.2) (end 140.65 89.4) (width 0.2) (layer F.Cu) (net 16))
 (segment (start 140.8 89.55) (end 141.939999 89.550001) (width 0.2) (layer F.Cu) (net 16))
 (segment (start 140.87377 89.550001) (end 140.8 89.55) (width 0.2) (layer F.Cu) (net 16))
 (via (at 143.6 90.2) (size 0.8) (drill 0.4) (layers F.Cu B.Cu) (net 10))
 (segment (start 144.6 90.2) (end 143.6 90.2) (width 0.2) (layer F.Cu) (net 10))
 (segment (start 143.3 90.2) (end 142.85 89.75) (width 0.2) (layer B.Cu) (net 10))
 (segment (start 143.6 90.2) (end 143.3 90.2) (width 0.2) (layer B.Cu) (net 10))
 (segment (start 146.075 90.2) (end 146.4 90.525) (width 0.2) (layer F.Cu) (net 10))
 (segment (start 144.6 90.2) (end 146.075 90.2) (width 0.2) (layer F.Cu) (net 10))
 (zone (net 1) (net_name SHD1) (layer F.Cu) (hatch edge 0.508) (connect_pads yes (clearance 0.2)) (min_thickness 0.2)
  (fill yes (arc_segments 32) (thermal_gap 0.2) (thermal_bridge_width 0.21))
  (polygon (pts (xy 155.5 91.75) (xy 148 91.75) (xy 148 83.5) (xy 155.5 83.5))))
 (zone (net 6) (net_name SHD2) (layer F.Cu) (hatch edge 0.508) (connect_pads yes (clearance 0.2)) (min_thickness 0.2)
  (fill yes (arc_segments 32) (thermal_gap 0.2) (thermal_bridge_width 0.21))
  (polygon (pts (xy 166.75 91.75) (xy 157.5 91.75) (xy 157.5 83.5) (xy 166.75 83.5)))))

